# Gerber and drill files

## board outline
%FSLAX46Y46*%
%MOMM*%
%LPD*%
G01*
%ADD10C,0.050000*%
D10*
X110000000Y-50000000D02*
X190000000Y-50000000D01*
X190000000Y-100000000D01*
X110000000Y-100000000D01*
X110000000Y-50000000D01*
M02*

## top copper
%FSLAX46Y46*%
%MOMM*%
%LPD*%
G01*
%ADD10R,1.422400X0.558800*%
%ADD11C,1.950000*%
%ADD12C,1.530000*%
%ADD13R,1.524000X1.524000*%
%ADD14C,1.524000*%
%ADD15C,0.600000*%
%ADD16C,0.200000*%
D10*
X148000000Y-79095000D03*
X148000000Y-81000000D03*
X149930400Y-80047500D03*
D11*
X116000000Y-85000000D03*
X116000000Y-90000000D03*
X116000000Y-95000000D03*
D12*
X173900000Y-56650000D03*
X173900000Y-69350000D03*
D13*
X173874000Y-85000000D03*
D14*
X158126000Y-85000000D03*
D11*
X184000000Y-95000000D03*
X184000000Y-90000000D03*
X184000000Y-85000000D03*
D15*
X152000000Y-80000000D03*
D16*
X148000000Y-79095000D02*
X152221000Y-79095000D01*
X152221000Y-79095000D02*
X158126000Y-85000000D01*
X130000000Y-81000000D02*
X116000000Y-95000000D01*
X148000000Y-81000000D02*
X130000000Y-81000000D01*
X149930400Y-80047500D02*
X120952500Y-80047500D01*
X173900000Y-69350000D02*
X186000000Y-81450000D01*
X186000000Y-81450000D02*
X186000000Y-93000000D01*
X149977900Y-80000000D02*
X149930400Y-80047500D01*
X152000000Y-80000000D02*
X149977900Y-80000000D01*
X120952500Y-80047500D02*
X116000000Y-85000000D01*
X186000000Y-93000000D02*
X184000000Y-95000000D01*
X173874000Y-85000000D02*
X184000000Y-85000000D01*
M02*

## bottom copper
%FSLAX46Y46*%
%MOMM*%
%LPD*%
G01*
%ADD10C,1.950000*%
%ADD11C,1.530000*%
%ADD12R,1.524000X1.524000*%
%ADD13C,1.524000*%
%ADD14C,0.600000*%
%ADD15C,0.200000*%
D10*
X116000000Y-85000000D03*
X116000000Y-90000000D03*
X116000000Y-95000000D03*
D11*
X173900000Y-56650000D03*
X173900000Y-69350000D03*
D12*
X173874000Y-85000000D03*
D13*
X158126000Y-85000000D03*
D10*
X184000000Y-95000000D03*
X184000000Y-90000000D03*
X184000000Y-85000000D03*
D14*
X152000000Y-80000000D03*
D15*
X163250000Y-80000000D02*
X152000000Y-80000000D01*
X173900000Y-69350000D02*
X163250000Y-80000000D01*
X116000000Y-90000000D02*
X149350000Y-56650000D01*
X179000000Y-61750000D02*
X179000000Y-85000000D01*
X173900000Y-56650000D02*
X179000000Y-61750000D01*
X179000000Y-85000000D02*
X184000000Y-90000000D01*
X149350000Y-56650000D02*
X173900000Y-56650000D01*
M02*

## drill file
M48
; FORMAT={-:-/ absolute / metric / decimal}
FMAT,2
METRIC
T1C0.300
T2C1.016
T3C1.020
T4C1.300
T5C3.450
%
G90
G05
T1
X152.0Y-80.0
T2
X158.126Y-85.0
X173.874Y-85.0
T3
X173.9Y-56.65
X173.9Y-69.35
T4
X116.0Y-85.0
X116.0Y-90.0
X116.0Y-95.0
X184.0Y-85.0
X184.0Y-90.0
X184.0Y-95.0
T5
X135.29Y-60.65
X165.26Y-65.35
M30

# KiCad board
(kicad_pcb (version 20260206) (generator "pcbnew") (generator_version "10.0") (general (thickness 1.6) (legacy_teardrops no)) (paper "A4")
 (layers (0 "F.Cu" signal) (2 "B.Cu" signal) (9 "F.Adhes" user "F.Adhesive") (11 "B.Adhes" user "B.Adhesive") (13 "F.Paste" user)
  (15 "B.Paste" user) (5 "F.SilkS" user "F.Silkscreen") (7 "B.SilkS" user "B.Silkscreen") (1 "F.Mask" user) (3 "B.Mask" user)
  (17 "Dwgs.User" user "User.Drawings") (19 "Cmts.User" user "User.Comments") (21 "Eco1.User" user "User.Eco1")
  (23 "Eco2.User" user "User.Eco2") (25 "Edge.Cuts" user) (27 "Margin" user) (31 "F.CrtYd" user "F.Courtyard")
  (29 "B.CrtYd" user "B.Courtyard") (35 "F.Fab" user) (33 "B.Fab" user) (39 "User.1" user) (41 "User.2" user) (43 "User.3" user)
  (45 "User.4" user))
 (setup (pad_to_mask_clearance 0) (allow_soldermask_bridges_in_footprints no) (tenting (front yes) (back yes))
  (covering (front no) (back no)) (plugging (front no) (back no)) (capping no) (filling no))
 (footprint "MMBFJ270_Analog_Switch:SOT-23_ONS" (layer "F.Cu") (at 148.9652 80.0475 -90)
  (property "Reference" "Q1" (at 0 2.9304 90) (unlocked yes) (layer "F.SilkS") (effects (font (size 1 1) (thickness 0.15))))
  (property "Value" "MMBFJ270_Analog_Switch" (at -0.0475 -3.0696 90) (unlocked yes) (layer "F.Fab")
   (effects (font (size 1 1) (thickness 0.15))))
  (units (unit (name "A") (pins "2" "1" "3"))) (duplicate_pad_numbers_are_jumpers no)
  (pad "1" smd rect (at -0.9525 0.9652 270) (size 0.5588 1.4224) (layers "F.Cu" "F.Mask" "F.Paste") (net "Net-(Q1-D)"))
  (pad "2" smd rect (at 0.9525 0.9652 270) (size 0.5588 1.4224) (layers "F.Cu" "F.Mask" "F.Paste") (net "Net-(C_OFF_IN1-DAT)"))
  (pad "3" smd rect (at 0 -0.9652 270) (size 0.5588 1.4224) (layers "F.Cu" "F.Mask" "F.Paste") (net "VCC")))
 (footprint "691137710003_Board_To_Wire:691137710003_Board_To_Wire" (layer "F.Cu") (at 116 90 -90)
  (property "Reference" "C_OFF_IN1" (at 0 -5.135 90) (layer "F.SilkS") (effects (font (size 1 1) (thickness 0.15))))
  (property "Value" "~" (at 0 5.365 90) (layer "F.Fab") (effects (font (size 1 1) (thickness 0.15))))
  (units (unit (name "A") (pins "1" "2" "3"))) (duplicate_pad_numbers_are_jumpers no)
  (pad "1" thru_hole circle (at -5 0 270) (size 1.95 1.95) (drill 1.3) (layers "*.Cu" "*.Mask") (remove_unused_layers no) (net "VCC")
   (solder_mask_margin 0.102))
  (pad "2" thru_hole circle (at 0 0 270) (size 1.95 1.95) (drill 1.3) (layers "*.Cu" "*.Mask") (remove_unused_layers no) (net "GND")
   (solder_mask_margin 0.102))
  (pad "3" thru_hole circle (at 5 0 270) (size 1.95 1.95) (drill 1.3) (layers "*.Cu" "*.Mask") (remove_unused_layers no)
   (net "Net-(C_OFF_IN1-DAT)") (solder_mask_margin 0.102)))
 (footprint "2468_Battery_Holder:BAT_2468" (layer "F.Cu") (at 150 63)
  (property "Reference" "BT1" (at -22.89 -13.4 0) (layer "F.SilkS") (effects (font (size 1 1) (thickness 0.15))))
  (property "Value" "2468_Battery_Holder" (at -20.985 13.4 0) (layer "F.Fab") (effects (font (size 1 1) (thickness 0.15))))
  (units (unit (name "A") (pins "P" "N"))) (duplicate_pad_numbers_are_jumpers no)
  (pad "" np_thru_hole circle (at -14.71 -2.35) (size 3.45 3.45) (drill 3.45) (layers "*.Cu" "*.Mask"))
  (pad "" np_thru_hole circle (at 15.26 2.35) (size 3.45 3.45) (drill 3.45) (layers "*.Cu" "*.Mask"))
  (pad "N" thru_hole circle (at 23.9 -6.35) (size 1.53 1.53) (drill 1.02) (layers "*.Cu" "*.Mask") (remove_unused_layers no) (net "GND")
   (solder_mask_margin 0.102))
  (pad "P" thru_hole circle (at 23.9 6.35) (size 1.53 1.53) (drill 1.02) (layers "*.Cu" "*.Mask") (remove_unused_layers no) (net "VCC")
   (solder_mask_margin 0.102)))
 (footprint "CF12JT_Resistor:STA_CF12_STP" (layer "F.Cu") (at 173.874 85 180)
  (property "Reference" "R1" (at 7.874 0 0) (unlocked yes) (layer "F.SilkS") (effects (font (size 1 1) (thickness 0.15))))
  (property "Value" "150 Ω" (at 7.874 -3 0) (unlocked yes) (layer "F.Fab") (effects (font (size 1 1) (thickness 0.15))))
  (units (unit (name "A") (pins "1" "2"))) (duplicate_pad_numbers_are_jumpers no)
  (pad "1" thru_hole rect (at 0 0 180) (size 1.524 1.524) (drill 1.016) (layers "*.Cu" "*.Mask") (remove_unused_layers no)
   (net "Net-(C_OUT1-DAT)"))
  (pad "2" thru_hole circle (at 15.748 0 180) (size 1.524 1.524) (drill 1.016) (layers "*.Cu" "*.Mask") (remove_unused_layers no)
   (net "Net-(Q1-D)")))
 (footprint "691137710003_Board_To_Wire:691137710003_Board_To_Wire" (layer "F.Cu") (at 184 90 90)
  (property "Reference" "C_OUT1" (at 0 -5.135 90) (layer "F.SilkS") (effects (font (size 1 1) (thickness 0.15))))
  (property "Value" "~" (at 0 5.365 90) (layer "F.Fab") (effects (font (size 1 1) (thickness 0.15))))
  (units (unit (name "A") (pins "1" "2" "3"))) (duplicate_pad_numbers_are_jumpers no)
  (pad "1" thru_hole circle (at -5 0 90) (size 1.95 1.95) (drill 1.3) (layers "*.Cu" "*.Mask") (remove_unused_layers no) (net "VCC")
   (solder_mask_margin 0.102))
  (pad "2" thru_hole circle (at 0 0 90) (size 1.95 1.95) (drill 1.3) (layers "*.Cu" "*.Mask") (remove_unused_layers no) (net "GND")
   (solder_mask_margin 0.102))
  (pad "3" thru_hole circle (at 5 0 90) (size 1.95 1.95) (drill 1.3) (layers "*.Cu" "*.Mask") (remove_unused_layers no)
   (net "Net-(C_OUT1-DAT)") (solder_mask_margin 0.102)))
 (gr_rect (start 110 50) (end 190 100) (stroke (width 0.05) (type default)) (fill no) (layer "Edge.Cuts"))
 (segment (start 148 79.095) (end 152.221 79.095) (width 0.2) (layer "F.Cu") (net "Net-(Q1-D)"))
 (segment (start 152.221 79.095) (end 158.126 85) (width 0.2) (layer "F.Cu") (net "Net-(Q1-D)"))
 (segment (start 130 81) (end 116 95) (width 0.2) (layer "F.Cu") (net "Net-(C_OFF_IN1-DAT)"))
 (segment (start 148 81) (end 130 81) (width 0.2) (layer "F.Cu") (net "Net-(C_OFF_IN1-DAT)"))
 (segment (start 149.9304 80.0475) (end 120.9525 80.0475) (width 0.2) (layer "F.Cu") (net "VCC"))
 (segment (start 173.9 69.35) (end 186 81.45) (width 0.2) (layer "F.Cu") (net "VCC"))
 (segment (start 186 81.45) (end 186 93) (width 0.2) (layer "F.Cu") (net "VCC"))
 (segment (start 149.9779 80) (end 149.9304 80.0475) (width 0.2) (layer "F.Cu") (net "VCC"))
 (segment (start 152 80) (end 149.9779 80) (width 0.2) (layer "F.Cu") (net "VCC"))
 (segment (start 120.9525 80.0475) (end 116 85) (width 0.2) (layer "F.Cu") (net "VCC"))
 (segment (start 186 93) (end 184 95) (width 0.2) (layer "F.Cu") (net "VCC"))
 (via (at 152 80) (size 0.6) (drill 0.3) (layers "F.Cu" "B.Cu") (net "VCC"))
 (segment (start 163.25 80) (end 152 80) (width 0.2) (layer "B.Cu") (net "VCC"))
 (segment (start 173.9 69.35) (end 163.25 80) (width 0.2) (layer "B.Cu") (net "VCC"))
 (segment (start 116 90) (end 149.35 56.65) (width 0.2) (layer "B.Cu") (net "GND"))
 (segment (start 179 61.75) (end 179 85) (width 0.2) (layer "B.Cu") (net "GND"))
 (segment (start 173.9 56.65) (end 179 61.75) (width 0.2) (layer "B.Cu") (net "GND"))
 (segment (start 179 85) (end 184 90) (width 0.2) (layer "B.Cu") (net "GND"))
 (segment (start 149.35 56.65) (end 173.9 56.65) (width 0.2) (layer "B.Cu") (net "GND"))
 (segment (start 173.874 85) (end 184 85) (width 0.2) (layer "F.Cu") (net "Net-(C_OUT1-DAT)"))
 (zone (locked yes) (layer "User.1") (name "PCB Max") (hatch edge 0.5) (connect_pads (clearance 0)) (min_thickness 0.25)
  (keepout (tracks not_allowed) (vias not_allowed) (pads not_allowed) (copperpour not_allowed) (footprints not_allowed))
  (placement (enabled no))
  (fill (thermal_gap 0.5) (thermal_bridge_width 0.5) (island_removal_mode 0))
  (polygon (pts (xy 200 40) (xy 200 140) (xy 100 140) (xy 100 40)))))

